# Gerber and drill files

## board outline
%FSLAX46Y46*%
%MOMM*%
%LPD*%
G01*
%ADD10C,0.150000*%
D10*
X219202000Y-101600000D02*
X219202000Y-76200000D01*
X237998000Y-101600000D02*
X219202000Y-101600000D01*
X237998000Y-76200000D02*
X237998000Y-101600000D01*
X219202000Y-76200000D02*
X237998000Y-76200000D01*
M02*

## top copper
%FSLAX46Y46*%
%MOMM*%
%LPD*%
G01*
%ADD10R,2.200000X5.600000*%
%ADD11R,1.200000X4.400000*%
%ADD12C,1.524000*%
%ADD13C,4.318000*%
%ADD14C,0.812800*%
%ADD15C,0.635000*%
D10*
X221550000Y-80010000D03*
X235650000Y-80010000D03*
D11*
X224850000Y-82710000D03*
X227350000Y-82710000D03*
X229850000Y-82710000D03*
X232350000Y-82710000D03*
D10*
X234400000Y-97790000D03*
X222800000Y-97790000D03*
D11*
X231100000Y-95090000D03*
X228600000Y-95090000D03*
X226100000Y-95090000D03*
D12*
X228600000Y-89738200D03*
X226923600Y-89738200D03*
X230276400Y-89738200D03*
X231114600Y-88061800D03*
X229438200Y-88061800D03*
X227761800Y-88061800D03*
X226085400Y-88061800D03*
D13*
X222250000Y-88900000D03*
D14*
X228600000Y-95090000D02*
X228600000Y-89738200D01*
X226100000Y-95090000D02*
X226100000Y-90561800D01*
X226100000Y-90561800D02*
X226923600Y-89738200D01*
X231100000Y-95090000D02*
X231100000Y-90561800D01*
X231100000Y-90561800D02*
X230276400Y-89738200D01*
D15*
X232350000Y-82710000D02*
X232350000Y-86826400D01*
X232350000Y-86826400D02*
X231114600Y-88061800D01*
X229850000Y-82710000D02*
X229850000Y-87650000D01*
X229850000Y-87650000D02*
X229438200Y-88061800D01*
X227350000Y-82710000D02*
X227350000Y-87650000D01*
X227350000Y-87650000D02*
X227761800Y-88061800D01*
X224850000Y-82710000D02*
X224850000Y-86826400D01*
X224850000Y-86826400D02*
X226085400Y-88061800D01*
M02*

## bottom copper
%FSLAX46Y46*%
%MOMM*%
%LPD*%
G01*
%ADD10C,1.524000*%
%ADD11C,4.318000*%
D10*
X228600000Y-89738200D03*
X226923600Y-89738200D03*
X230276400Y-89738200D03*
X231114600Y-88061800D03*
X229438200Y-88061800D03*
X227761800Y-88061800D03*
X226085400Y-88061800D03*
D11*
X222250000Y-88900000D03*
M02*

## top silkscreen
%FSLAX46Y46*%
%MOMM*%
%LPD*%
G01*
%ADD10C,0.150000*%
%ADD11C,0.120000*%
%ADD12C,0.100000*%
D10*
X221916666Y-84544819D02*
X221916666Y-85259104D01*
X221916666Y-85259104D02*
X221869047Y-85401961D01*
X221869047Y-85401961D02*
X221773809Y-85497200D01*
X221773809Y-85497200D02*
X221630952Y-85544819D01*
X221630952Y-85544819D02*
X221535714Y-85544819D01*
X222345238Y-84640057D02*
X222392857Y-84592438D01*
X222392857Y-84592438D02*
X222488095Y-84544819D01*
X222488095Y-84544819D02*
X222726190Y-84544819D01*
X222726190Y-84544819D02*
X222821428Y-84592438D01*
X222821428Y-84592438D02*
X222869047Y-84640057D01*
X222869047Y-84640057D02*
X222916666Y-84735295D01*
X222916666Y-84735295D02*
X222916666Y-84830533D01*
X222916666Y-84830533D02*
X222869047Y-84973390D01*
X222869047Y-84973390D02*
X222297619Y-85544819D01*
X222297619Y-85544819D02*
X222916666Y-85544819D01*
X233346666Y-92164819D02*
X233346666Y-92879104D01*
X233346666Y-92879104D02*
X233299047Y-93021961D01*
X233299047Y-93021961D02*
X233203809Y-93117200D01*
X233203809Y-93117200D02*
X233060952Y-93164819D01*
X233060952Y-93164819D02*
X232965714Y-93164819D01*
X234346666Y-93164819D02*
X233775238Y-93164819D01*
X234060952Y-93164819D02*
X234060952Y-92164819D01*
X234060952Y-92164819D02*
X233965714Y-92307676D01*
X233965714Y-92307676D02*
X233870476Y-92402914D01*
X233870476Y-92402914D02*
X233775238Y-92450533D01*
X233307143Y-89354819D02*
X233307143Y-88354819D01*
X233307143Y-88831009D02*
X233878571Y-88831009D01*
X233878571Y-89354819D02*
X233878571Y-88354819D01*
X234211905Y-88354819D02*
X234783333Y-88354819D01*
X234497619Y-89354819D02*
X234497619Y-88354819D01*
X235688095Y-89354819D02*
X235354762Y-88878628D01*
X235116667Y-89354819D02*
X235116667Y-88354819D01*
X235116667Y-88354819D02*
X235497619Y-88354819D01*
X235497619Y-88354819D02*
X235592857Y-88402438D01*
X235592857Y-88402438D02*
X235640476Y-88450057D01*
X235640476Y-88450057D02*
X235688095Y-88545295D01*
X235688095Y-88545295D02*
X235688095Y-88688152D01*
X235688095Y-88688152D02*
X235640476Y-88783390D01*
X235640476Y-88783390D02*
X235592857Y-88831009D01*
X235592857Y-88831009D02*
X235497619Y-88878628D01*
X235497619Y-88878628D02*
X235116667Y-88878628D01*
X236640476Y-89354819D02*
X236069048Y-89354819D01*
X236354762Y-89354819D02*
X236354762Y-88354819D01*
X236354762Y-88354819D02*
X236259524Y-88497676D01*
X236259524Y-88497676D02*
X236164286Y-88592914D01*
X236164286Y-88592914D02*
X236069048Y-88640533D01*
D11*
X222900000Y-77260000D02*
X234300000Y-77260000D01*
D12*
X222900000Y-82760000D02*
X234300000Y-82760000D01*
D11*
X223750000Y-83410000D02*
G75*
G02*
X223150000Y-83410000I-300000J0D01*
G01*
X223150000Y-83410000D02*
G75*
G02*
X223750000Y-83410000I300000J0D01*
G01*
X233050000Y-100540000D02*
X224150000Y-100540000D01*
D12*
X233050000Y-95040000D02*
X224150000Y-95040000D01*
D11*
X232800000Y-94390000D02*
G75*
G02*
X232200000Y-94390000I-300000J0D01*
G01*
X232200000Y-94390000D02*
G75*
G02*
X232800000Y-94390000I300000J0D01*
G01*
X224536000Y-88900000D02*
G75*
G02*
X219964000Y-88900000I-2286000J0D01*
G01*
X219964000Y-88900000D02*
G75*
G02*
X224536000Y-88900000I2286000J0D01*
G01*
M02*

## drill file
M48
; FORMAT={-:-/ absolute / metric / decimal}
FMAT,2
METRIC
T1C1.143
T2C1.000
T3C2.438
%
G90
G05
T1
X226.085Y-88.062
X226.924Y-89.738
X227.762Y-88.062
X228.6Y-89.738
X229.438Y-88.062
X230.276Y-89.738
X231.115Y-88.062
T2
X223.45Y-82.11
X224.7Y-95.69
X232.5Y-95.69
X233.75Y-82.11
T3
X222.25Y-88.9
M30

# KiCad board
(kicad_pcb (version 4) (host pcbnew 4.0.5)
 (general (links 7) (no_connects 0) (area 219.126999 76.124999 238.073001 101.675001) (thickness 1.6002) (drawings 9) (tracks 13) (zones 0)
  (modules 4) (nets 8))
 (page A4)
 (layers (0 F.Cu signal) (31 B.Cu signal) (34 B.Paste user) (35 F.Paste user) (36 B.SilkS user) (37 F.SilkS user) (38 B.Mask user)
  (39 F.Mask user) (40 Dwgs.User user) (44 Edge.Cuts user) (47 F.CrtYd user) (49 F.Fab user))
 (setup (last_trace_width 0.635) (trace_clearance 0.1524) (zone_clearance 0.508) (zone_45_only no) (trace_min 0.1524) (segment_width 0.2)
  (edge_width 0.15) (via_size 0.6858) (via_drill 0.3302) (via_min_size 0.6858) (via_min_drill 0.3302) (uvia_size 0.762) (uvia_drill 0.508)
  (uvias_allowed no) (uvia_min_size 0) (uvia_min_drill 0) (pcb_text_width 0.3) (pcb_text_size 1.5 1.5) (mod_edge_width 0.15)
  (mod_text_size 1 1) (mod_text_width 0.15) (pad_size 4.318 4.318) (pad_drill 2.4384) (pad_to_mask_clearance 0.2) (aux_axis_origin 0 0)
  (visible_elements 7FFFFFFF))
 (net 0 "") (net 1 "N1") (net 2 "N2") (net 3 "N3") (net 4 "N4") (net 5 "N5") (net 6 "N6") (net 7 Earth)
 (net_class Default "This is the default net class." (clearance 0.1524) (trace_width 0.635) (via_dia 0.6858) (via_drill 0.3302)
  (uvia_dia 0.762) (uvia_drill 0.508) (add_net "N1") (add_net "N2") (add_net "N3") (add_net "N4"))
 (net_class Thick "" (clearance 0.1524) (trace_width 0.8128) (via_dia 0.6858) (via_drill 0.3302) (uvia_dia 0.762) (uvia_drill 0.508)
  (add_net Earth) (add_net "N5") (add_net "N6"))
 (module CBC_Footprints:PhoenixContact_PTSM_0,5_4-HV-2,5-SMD (layer F.Cu) (at 228.6 80.01)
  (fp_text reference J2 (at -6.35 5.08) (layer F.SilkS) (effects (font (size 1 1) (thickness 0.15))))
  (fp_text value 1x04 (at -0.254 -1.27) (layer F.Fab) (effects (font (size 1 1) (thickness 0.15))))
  (fp_line (start -5.7 -2.75) (end 5.7 -2.75) (layer F.SilkS) (width 0.12))
  (fp_line (start -5.7 2.75) (end 5.7 2.75) (layer F.SilkS) (width 0.1))
  (fp_circle (center -5.15 3.4) (end -5.45 3.4) (layer F.SilkS) (width 0.12))
  (pad "" smd rect (at -7.05 0) (size 2.2 5.6) (layers F.Cu F.Paste F.Mask))
  (pad "" smd rect (at 7.05 0) (size 2.2 5.6) (layers F.Cu F.Paste F.Mask))
  (pad 1 smd rect (at -3.75 2.7) (size 1.2 4.4) (layers F.Cu F.Paste F.Mask) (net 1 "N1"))
  (pad 2 smd rect (at -1.25 2.7) (size 1.2 4.4) (layers F.Cu F.Paste F.Mask) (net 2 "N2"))
  (pad 3 smd rect (at 1.25 2.7) (size 1.2 4.4) (layers F.Cu F.Paste F.Mask) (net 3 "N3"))
  (pad 4 smd rect (at 3.75 2.7) (size 1.2 4.4) (layers F.Cu F.Paste F.Mask) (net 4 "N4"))
  (pad "" np_thru_hole circle (at -5.15 2.1) (size 1 1) (drill 1) (layers *.Cu *.Mask))
  (pad "" np_thru_hole circle (at 5.15 2.1) (size 1 1) (drill 1) (layers *.Cu *.Mask)))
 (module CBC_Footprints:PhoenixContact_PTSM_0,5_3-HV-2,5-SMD (layer F.Cu) (at 228.6 97.79 180)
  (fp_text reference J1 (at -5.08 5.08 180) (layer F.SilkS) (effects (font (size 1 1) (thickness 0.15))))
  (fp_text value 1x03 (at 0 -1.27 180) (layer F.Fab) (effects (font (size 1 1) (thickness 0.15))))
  (fp_line (start -4.45 -2.75) (end 4.45 -2.75) (layer F.SilkS) (width 0.12))
  (fp_line (start -4.45 2.75) (end 4.45 2.75) (layer F.SilkS) (width 0.1))
  (fp_circle (center -3.9 3.4) (end -4.2 3.4) (layer F.SilkS) (width 0.12))
  (pad "" smd rect (at -5.8 0 180) (size 2.2 5.6) (layers F.Cu F.Paste F.Mask))
  (pad "" smd rect (at 5.8 0 180) (size 2.2 5.6) (layers F.Cu F.Paste F.Mask))
  (pad 1 smd rect (at -2.5 2.7 180) (size 1.2 4.4) (layers F.Cu F.Paste F.Mask) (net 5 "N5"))
  (pad 2 smd rect (at 0 2.7 180) (size 1.2 4.4) (layers F.Cu F.Paste F.Mask) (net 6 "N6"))
  (pad 3 smd rect (at 2.5 2.7 180) (size 1.2 4.4) (layers F.Cu F.Paste F.Mask) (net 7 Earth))
  (pad "" np_thru_hole circle (at -3.9 2.1 180) (size 1 1) (drill 1) (layers *.Cu *.Mask))
  (pad "" np_thru_hole circle (at 3.9 2.1 180) (size 1 1) (drill 1) (layers *.Cu *.Mask)))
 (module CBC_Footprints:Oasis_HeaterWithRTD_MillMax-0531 (layer F.Cu) (at 228.6 88.9)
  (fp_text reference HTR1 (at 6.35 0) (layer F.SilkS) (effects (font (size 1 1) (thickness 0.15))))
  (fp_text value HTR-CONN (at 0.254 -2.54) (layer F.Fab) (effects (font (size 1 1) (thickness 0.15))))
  (pad 2 thru_hole circle (at 0 0.8382) (size 1.524 1.524) (drill 1.143) (layers *.Cu *.Mask) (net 6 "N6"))
  (pad 3 thru_hole circle (at -1.6764 0.8382) (size 1.524 1.524) (drill 1.143) (layers *.Cu *.Mask) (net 7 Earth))
  (pad 1 thru_hole circle (at 1.6764 0.8382) (size 1.524 1.524) (drill 1.143) (layers *.Cu *.Mask) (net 5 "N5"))
  (pad 7 thru_hole circle (at 2.5146 -0.8382) (size 1.524 1.524) (drill 1.143) (layers *.Cu *.Mask) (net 4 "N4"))
  (pad 6 thru_hole circle (at 0.8382 -0.8382) (size 1.524 1.524) (drill 1.143) (layers *.Cu *.Mask) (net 3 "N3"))
  (pad 5 thru_hole circle (at -0.8382 -0.8382) (size 1.524 1.524) (drill 1.143) (layers *.Cu *.Mask) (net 2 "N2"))
  (pad 4 thru_hole circle (at -2.5146 -0.8382) (size 1.524 1.524) (drill 1.143) (layers *.Cu *.Mask) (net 1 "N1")))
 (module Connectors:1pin (layer F.Cu) (at 222.25 88.9)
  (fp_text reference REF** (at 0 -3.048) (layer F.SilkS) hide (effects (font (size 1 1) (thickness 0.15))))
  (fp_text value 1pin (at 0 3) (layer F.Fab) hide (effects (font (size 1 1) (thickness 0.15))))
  (fp_circle (center 0 0) (end 0 -2.286) (layer F.SilkS) (width 0.12))
  (pad "" np_thru_hole circle (at 0 0) (size 4.318 4.318) (drill 2.4384) (layers *.Cu *.Mask)))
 (gr_line (start 219.202 101.6) (end 219.202 76.2) (angle 90) (layer Edge.Cuts) (width 0.15))
 (gr_line (start 237.998 101.6) (end 219.202 101.6) (angle 90) (layer Edge.Cuts) (width 0.15))
 (gr_line (start 237.998 76.2) (end 237.998 101.6) (angle 90) (layer Edge.Cuts) (width 0.15))
 (gr_line (start 219.202 76.2) (end 237.998 76.2) (angle 90) (layer Edge.Cuts) (width 0.15))
 (segment (start 228.6 95.09) (end 228.6 89.7382) (width 0.8128) (layer F.Cu) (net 6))
 (segment (start 226.1 95.09) (end 226.1 90.5618) (width 0.8128) (layer F.Cu) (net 7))
 (segment (start 226.1 90.5618) (end 226.9236 89.7382) (width 0.8128) (layer F.Cu) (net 7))
 (segment (start 231.1 95.09) (end 231.1 90.5618) (width 0.8128) (layer F.Cu) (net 5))
 (segment (start 231.1 90.5618) (end 230.2764 89.7382) (width 0.8128) (layer F.Cu) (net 5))
 (segment (start 232.35 82.71) (end 232.35 86.8264) (width 0.635) (layer F.Cu) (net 4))
 (segment (start 232.35 86.8264) (end 231.1146 88.0618) (width 0.635) (layer F.Cu) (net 4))
 (segment (start 229.85 82.71) (end 229.85 87.65) (width 0.635) (layer F.Cu) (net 3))
 (segment (start 229.85 87.65) (end 229.4382 88.0618) (width 0.635) (layer F.Cu) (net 3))
 (segment (start 227.35 82.71) (end 227.35 87.65) (width 0.635) (layer F.Cu) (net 2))
 (segment (start 227.35 87.65) (end 227.7618 88.0618) (width 0.635) (layer F.Cu) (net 2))
 (segment (start 224.85 82.71) (end 224.85 86.8264) (width 0.635) (layer F.Cu) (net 1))
 (segment (start 224.85 86.8264) (end 226.0854 88.0618) (width 0.635) (layer F.Cu) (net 1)))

